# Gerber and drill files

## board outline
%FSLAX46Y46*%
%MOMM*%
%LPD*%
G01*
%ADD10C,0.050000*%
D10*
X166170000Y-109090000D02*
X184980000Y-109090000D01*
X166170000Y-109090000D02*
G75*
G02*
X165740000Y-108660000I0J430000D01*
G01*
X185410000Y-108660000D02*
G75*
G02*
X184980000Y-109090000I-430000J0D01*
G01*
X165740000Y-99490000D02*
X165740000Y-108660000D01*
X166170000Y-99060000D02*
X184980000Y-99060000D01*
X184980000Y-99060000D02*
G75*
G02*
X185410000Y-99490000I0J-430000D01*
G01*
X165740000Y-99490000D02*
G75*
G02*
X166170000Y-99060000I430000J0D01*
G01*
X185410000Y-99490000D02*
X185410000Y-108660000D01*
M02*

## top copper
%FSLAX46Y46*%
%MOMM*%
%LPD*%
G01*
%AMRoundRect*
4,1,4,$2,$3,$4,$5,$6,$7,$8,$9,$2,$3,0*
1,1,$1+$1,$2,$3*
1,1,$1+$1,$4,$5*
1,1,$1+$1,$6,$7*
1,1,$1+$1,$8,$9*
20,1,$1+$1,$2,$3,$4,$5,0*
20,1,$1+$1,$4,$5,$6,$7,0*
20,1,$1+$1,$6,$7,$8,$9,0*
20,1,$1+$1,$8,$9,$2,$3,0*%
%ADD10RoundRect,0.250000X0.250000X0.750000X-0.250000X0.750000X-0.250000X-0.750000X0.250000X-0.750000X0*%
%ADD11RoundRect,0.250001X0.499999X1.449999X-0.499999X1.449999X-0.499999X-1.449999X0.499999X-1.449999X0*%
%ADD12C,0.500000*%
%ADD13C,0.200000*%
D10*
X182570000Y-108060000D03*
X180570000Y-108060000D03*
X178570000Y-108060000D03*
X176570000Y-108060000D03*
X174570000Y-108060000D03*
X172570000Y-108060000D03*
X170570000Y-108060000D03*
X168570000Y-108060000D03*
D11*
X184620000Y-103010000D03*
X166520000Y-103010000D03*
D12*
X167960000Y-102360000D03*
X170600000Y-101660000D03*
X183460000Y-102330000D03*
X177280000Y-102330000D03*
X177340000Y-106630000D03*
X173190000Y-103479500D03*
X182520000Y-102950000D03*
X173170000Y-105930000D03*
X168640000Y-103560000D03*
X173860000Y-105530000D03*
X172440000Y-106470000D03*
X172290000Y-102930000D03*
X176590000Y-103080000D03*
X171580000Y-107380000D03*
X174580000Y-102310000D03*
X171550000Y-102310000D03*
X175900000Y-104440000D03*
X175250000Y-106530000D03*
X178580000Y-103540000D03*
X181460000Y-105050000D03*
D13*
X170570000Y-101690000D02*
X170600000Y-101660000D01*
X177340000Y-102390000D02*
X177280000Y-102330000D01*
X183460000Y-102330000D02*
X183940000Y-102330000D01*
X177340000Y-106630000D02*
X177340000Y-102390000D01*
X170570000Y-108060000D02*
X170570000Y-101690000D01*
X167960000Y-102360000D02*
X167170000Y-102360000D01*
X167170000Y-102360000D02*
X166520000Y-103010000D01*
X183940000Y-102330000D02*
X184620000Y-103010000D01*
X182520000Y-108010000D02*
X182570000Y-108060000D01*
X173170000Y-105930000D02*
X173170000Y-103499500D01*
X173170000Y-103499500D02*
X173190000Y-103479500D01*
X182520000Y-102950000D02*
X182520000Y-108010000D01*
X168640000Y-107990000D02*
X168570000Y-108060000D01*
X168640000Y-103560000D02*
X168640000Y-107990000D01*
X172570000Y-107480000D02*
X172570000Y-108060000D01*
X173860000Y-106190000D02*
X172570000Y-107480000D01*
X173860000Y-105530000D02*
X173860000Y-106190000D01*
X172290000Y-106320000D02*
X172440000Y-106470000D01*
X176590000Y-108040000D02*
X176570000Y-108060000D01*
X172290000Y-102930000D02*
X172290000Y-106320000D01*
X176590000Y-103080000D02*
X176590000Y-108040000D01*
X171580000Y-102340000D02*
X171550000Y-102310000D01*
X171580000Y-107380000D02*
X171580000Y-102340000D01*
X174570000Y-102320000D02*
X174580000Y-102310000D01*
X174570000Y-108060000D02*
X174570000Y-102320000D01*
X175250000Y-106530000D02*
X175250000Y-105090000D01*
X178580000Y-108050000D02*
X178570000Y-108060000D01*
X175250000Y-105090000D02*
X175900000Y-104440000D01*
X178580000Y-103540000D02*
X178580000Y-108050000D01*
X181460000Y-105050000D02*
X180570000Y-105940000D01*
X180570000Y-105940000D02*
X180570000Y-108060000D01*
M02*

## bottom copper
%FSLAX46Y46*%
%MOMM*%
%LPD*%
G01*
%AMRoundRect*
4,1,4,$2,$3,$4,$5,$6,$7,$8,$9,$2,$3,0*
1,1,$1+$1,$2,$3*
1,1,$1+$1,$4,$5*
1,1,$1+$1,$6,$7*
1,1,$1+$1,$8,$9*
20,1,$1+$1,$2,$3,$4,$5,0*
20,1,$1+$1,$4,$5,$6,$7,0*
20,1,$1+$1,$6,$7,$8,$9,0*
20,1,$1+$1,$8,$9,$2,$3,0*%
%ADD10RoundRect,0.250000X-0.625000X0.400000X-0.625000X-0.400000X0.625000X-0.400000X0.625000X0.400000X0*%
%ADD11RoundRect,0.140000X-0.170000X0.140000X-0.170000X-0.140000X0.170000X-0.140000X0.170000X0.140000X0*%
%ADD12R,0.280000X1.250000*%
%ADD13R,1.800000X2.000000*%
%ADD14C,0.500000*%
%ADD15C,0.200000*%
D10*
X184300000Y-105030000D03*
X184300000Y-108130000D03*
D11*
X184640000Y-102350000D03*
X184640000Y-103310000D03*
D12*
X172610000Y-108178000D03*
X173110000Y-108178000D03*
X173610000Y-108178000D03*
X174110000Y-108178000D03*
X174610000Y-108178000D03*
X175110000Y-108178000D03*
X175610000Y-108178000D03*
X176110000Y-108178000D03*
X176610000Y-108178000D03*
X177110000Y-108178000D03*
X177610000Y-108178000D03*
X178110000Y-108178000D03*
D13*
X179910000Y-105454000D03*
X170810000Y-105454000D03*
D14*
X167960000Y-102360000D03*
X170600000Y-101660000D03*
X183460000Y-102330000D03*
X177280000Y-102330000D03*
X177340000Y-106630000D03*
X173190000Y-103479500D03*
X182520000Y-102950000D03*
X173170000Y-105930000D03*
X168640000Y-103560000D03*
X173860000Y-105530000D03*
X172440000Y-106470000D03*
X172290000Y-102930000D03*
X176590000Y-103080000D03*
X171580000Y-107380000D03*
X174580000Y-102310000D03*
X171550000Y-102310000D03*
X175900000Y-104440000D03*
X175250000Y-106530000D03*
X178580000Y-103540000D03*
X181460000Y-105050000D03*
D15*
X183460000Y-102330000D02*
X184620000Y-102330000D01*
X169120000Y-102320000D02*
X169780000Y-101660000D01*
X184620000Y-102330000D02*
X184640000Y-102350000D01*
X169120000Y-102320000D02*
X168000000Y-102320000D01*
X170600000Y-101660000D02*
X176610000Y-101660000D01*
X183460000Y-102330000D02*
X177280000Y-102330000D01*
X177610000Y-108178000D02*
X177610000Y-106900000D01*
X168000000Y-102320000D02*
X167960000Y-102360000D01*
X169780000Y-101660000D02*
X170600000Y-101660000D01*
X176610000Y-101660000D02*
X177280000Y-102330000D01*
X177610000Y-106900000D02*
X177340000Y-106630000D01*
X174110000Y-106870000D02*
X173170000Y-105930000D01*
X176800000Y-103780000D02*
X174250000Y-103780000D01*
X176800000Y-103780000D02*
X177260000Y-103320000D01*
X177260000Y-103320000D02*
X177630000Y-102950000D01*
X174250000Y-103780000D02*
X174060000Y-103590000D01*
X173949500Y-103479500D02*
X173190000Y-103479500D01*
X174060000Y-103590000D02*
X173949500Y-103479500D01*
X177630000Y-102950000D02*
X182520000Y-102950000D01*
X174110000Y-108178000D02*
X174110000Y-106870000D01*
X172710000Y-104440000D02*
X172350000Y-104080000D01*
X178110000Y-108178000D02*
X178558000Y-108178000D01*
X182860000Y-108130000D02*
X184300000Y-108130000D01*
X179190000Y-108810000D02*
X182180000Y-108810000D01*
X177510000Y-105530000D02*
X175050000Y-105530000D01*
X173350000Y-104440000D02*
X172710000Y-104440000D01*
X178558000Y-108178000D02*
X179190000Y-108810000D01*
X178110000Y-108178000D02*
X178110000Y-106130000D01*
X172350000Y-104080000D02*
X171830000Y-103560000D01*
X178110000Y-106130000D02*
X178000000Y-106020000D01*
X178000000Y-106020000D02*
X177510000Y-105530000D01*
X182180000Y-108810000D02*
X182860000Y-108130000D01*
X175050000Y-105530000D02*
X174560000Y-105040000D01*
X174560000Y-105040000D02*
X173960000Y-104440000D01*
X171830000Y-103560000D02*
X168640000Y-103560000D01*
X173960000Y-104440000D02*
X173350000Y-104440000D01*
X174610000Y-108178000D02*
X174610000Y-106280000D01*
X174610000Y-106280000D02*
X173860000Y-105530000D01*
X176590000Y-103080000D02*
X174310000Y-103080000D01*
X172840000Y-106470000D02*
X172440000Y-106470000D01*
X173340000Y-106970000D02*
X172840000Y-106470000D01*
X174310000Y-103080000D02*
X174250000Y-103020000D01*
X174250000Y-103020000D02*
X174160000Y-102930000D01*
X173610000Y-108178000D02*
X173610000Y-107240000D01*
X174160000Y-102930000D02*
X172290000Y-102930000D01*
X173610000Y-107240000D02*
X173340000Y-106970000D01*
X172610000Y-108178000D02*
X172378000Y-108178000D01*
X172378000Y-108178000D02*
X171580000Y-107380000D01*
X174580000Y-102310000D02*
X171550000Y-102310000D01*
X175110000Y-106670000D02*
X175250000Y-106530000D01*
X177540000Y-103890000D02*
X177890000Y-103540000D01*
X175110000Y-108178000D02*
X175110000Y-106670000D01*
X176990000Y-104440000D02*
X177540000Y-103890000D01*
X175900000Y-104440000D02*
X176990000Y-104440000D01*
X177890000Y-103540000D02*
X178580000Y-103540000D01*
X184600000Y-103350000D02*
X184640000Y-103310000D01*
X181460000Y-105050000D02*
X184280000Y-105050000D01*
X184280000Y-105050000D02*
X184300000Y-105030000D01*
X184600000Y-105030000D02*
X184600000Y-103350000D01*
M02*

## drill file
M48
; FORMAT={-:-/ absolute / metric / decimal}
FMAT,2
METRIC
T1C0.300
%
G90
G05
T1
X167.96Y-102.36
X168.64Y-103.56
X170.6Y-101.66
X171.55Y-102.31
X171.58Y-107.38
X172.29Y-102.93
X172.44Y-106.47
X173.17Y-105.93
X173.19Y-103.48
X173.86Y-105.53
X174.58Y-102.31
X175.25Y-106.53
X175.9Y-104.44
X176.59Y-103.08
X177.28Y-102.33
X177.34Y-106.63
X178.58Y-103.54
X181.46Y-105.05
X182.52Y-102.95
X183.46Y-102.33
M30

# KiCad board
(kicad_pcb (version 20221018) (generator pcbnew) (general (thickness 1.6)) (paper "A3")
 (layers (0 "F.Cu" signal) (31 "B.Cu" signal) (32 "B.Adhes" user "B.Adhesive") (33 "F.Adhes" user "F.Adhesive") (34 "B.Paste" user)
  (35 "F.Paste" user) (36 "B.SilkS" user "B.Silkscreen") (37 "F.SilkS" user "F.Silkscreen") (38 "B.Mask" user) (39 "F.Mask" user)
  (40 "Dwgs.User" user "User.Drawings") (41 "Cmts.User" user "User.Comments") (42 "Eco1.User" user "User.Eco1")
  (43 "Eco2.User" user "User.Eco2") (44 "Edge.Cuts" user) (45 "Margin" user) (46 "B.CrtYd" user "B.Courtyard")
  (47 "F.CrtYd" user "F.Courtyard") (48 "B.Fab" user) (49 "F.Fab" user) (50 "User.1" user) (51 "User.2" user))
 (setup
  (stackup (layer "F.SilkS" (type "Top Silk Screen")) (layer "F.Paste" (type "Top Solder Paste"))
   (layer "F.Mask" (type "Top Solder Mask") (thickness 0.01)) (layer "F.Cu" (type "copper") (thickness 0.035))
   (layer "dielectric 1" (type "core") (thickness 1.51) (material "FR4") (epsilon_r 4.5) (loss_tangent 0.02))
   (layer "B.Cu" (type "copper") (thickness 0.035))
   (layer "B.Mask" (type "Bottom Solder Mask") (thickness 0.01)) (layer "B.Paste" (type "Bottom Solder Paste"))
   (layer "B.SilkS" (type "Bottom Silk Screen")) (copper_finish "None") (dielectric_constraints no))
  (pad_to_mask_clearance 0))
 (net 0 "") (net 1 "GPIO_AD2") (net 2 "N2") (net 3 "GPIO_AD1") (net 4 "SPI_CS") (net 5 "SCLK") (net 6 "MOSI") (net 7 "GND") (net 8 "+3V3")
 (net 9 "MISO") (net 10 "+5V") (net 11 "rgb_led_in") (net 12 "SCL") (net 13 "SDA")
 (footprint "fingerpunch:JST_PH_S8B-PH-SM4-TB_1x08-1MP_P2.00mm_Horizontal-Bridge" (layer "F.Cu") (at 175.57 105.16 180)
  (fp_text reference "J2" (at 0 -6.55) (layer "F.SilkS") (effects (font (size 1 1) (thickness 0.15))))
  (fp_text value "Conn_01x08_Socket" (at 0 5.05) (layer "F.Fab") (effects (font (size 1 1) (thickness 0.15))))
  (pad "1" smd roundrect (at -7 -2.9 180) (size 1 2) (layers "F.Cu" "F.Paste" "F.Mask") (roundrect_rratio 0.25) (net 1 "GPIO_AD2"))
  (pad "2" smd roundrect (at -5 -2.9 180) (size 1 2) (layers "F.Cu" "F.Paste" "F.Mask") (roundrect_rratio 0.25) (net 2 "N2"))
  (pad "3" smd roundrect (at -3 -2.9 180) (size 1 2) (layers "F.Cu" "F.Paste" "F.Mask") (roundrect_rratio 0.25) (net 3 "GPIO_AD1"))
  (pad "4" smd roundrect (at -1 -2.9 180) (size 1 2) (layers "F.Cu" "F.Paste" "F.Mask") (roundrect_rratio 0.25) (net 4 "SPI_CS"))
  (pad "5" smd roundrect (at 1 -2.9 180) (size 1 2) (layers "F.Cu" "F.Paste" "F.Mask") (roundrect_rratio 0.25) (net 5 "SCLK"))
  (pad "6" smd roundrect (at 3 -2.9 180) (size 1 2) (layers "F.Cu" "F.Paste" "F.Mask") (roundrect_rratio 0.25) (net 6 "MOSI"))
  (pad "7" smd roundrect (at 5 -2.9 180) (size 1 2) (layers "F.Cu" "F.Paste" "F.Mask") (roundrect_rratio 0.25) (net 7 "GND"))
  (pad "8" smd roundrect (at 7 -2.9 180) (size 1 2) (layers "F.Cu" "F.Paste" "F.Mask") (roundrect_rratio 0.25) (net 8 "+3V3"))
  (pad "9" smd roundrect (at -9.05 2.15 180) (size 1.5 3.4) (layers "F.Cu" "F.Paste" "F.Mask") (roundrect_rratio 0.1666673333) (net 7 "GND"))
  (pad "9" smd roundrect (at 9.05 2.15 180) (size 1.5 3.4) (layers "F.Cu" "F.Paste" "F.Mask") (roundrect_rratio 0.1666673333) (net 7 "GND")))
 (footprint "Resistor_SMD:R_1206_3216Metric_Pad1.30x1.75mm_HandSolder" (layer "B.Cu") (at 184.3 106.58 -90)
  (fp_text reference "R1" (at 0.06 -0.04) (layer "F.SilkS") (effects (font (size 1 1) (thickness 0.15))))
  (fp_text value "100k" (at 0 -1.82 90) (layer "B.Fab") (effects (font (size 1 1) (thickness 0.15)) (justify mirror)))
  (pad "1" smd roundrect (at -1.55 0 270) (size 1.3 1.75) (layers "B.Cu" "B.Paste" "B.Mask") (roundrect_rratio 0.1923076923) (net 2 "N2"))
  (pad "2" smd roundrect (at 1.55 0 270) (size 1.3 1.75) (layers "B.Cu" "B.Paste" "B.Mask") (roundrect_rratio 0.1923076923) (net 8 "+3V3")))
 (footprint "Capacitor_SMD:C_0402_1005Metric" (layer "B.Cu") (at 184.64 102.83 -90)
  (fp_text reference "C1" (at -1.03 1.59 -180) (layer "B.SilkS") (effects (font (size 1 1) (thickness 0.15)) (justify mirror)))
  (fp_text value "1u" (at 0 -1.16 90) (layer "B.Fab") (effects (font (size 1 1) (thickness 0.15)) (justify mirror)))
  (pad "1" smd roundrect (at -0.48 0 270) (size 0.56 0.62) (layers "B.Cu" "B.Paste" "B.Mask") (roundrect_rratio 0.25) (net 7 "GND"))
  (pad "2" smd roundrect (at 0.48 0 270) (size 0.56 0.62) (layers "B.Cu" "B.Paste" "B.Mask") (roundrect_rratio 0.25) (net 2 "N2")))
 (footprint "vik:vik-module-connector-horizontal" (layer "B.Cu") (at 175.36 106.14)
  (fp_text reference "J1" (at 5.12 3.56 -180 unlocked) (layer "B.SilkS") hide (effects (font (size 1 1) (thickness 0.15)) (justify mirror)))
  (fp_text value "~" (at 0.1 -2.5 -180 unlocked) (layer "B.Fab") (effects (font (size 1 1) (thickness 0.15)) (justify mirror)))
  (pad "1" smd rect (at -2.75 2.038) (size 0.28 1.25) (layers "B.Cu" "B.Paste" "B.Mask") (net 5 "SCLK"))
  (pad "2" smd rect (at -2.25 2.038) (size 0.28 1.25) (layers "B.Cu" "B.Paste" "B.Mask") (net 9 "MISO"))
  (pad "3" smd rect (at -1.75 2.038) (size 0.28 1.25) (layers "B.Cu" "B.Paste" "B.Mask") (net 4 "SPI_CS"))
  (pad "4" smd rect (at -1.25 2.038) (size 0.28 1.25) (layers "B.Cu" "B.Paste" "B.Mask") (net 1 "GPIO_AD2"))
  (pad "5" smd rect (at -0.75 2.038) (size 0.28 1.25) (layers "B.Cu" "B.Paste" "B.Mask") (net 6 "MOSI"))
  (pad "6" smd rect (at -0.25 2.038) (size 0.28 1.25) (layers "B.Cu" "B.Paste" "B.Mask") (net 3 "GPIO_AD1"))
  (pad "7" smd rect (at 0.25 2.038) (size 0.28 1.25) (layers "B.Cu" "B.Paste" "B.Mask") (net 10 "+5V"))
  (pad "8" smd rect (at 0.75 2.038) (size 0.28 1.25) (layers "B.Cu" "B.Paste" "B.Mask") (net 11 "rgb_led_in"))
  (pad "9" smd rect (at 1.25 2.038) (size 0.28 1.25) (layers "B.Cu" "B.Paste" "B.Mask") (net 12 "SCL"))
  (pad "10" smd rect (at 1.75 2.038) (size 0.28 1.25) (layers "B.Cu" "B.Paste" "B.Mask") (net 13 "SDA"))
  (pad "11" smd rect (at 2.25 2.038) (size 0.28 1.25) (layers "B.Cu" "B.Paste" "B.Mask") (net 7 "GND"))
  (pad "12" smd rect (at 2.75 2.038) (size 0.28 1.25) (layers "B.Cu" "B.Paste" "B.Mask") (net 8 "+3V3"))
  (pad "13" smd rect (at 4.55 -0.686) (size 1.8 2) (layers "B.Cu" "B.Paste" "B.Mask"))
  (pad "14" smd rect (at -4.55 -0.686) (size 1.8 2) (layers "B.Cu" "B.Paste" "B.Mask")))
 (gr_line (start 166.17 109.09) (end 184.98 109.09) (stroke (width 0.05) (type default)) (layer "Edge.Cuts"))
 (gr_arc (start 166.17 109.09) (mid 165.865944 108.964056) (end 165.74 108.66) (stroke (width 0.05) (type default)) (layer "Edge.Cuts"))
 (gr_arc (start 185.41 108.66) (mid 185.284056 108.964056) (end 184.98 109.09) (stroke (width 0.05) (type default)) (layer "Edge.Cuts"))
 (gr_line (start 165.74 99.49) (end 165.74 108.66) (stroke (width 0.05) (type default)) (layer "Edge.Cuts"))
 (gr_line (start 166.17 99.06) (end 184.98 99.06) (stroke (width 0.05) (type default)) (layer "Edge.Cuts"))
 (gr_arc (start 184.98 99.06) (mid 185.284056 99.185944) (end 185.41 99.49) (stroke (width 0.05) (type default)) (layer "Edge.Cuts"))
 (gr_arc (start 165.74 99.49) (mid 165.865944 99.185944) (end 166.17 99.06) (stroke (width 0.05) (type default)) (layer "Edge.Cuts"))
 (gr_line (start 185.41 99.49) (end 185.41 108.66) (stroke (width 0.05) (type default)) (layer "Edge.Cuts"))
 (segment (start 170.57 101.69) (end 170.6 101.66) (width 0.2) (layer "F.Cu") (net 7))
 (segment (start 177.34 102.39) (end 177.28 102.33) (width 0.2) (layer "F.Cu") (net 7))
 (segment (start 183.46 102.33) (end 183.94 102.33) (width 0.2) (layer "F.Cu") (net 7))
 (segment (start 177.34 106.63) (end 177.34 102.39) (width 0.2) (layer "F.Cu") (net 7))
 (segment (start 170.57 108.06) (end 170.57 101.69) (width 0.2) (layer "F.Cu") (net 7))
 (segment (start 167.96 102.36) (end 167.17 102.36) (width 0.2) (layer "F.Cu") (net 7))
 (segment (start 167.17 102.36) (end 166.52 103.01) (width 0.2) (layer "F.Cu") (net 7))
 (segment (start 183.94 102.33) (end 184.62 103.01) (width 0.2) (layer "F.Cu") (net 7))
 (via (at 167.96 102.36) (size 0.5) (drill 0.3) (layers "F.Cu" "B.Cu") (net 7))
 (via (at 170.6 101.66) (size 0.5) (drill 0.3) (layers "F.Cu" "B.Cu") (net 7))
 (via (at 183.46 102.33) (size 0.5) (drill 0.3) (layers "F.Cu" "B.Cu") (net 7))
 (via (at 177.28 102.33) (size 0.5) (drill 0.3) (layers "F.Cu" "B.Cu") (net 7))
 (via (at 177.34 106.63) (size 0.5) (drill 0.3) (layers "F.Cu" "B.Cu") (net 7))
 (segment (start 183.46 102.33) (end 184.62 102.33) (width 0.2) (layer "B.Cu") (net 7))
 (segment (start 169.12 102.32) (end 169.78 101.66) (width 0.2) (layer "B.Cu") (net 7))
 (segment (start 184.62 102.33) (end 184.64 102.35) (width 0.2) (layer "B.Cu") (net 7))
 (segment (start 169.12 102.32) (end 168 102.32) (width 0.2) (layer "B.Cu") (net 7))
 (segment (start 170.6 101.66) (end 176.61 101.66) (width 0.2) (layer "B.Cu") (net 7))
 (segment (start 183.46 102.33) (end 177.28 102.33) (width 0.2) (layer "B.Cu") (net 7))
 (segment (start 177.61 108.178) (end 177.61 106.9) (width 0.2) (layer "B.Cu") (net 7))
 (segment (start 168 102.32) (end 167.96 102.36) (width 0.2) (layer "B.Cu") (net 7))
 (segment (start 169.78 101.66) (end 170.6 101.66) (width 0.2) (layer "B.Cu") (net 7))
 (segment (start 176.61 101.66) (end 177.28 102.33) (width 0.2) (layer "B.Cu") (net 7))
 (segment (start 177.61 106.9) (end 177.34 106.63) (width 0.2) (layer "B.Cu") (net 7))
 (segment (start 182.52 108.01) (end 182.57 108.06) (width 0.2) (layer "F.Cu") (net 1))
 (segment (start 173.17 105.93) (end 173.17 103.4995) (width 0.2) (layer "F.Cu") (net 1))
 (segment (start 173.17 103.4995) (end 173.19 103.4795) (width 0.2) (layer "F.Cu") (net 1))
 (segment (start 182.52 102.95) (end 182.52 108.01) (width 0.2) (layer "F.Cu") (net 1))
 (via (at 173.19 103.4795) (size 0.5) (drill 0.3) (layers "F.Cu" "B.Cu") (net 1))
 (via (at 182.52 102.95) (size 0.5) (drill 0.3) (layers "F.Cu" "B.Cu") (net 1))
 (via (at 173.17 105.93) (size 0.5) (drill 0.3) (layers "F.Cu" "B.Cu") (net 1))
 (segment (start 174.11 106.87) (end 173.17 105.93) (width 0.2) (layer "B.Cu") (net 1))
 (segment (start 176.8 103.78) (end 174.25 103.78) (width 0.2) (layer "B.Cu") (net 1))
 (segment (start 176.8 103.78) (end 177.26 103.32) (width 0.2) (layer "B.Cu") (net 1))
 (segment (start 177.26 103.32) (end 177.63 102.95) (width 0.2) (layer "B.Cu") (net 1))
 (segment (start 174.25 103.78) (end 174.06 103.59) (width 0.2) (layer "B.Cu") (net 1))
 (segment (start 173.9495 103.4795) (end 173.19 103.4795) (width 0.2) (layer "B.Cu") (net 1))
 (segment (start 174.06 103.59) (end 173.9495 103.4795) (width 0.2) (layer "B.Cu") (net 1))
 (segment (start 177.63 102.95) (end 182.52 102.95) (width 0.2) (layer "B.Cu") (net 1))
 (segment (start 174.11 108.178) (end 174.11 106.87) (width 0.2) (layer "B.Cu") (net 1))
 (segment (start 168.64 107.99) (end 168.57 108.06) (width 0.2) (layer "F.Cu") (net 8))
 (segment (start 168.64 103.56) (end 168.64 107.99) (width 0.2) (layer "F.Cu") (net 8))
 (via (at 168.64 103.56) (size 0.5) (drill 0.3) (layers "F.Cu" "B.Cu") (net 8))
 (segment (start 172.71 104.44) (end 172.35 104.08) (width 0.2) (layer "B.Cu") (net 8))
 (segment (start 178.11 108.178) (end 178.558 108.178) (width 0.2) (layer "B.Cu") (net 8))
 (segment (start 182.86 108.13) (end 184.3 108.13) (width 0.2) (layer "B.Cu") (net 8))
 (segment (start 179.19 108.81) (end 182.18 108.81) (width 0.2) (layer "B.Cu") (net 8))
 (segment (start 177.51 105.53) (end 175.05 105.53) (width 0.2) (layer "B.Cu") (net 8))
 (segment (start 173.35 104.44) (end 172.71 104.44) (width 0.2) (layer "B.Cu") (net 8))
 (segment (start 178.558 108.178) (end 179.19 108.81) (width 0.2) (layer "B.Cu") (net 8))
 (segment (start 178.11 108.178) (end 178.11 106.13) (width 0.2) (layer "B.Cu") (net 8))
 (segment (start 172.35 104.08) (end 171.83 103.56) (width 0.2) (layer "B.Cu") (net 8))
 (segment (start 178.11 106.13) (end 178 106.02) (width 0.2) (layer "B.Cu") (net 8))
 (segment (start 178 106.02) (end 177.51 105.53) (width 0.2) (layer "B.Cu") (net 8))
 (segment (start 182.18 108.81) (end 182.86 108.13) (width 0.2) (layer "B.Cu") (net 8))
 (segment (start 175.05 105.53) (end 174.56 105.04) (width 0.2) (layer "B.Cu") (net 8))
 (segment (start 174.56 105.04) (end 173.96 104.44) (width 0.2) (layer "B.Cu") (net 8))
 (segment (start 171.83 103.56) (end 168.64 103.56) (width 0.2) (layer "B.Cu") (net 8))
 (segment (start 173.96 104.44) (end 173.35 104.44) (width 0.2) (layer "B.Cu") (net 8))
 (segment (start 172.57 107.48) (end 172.57 108.06) (width 0.2) (layer "F.Cu") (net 6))
 (segment (start 173.86 106.19) (end 172.57 107.48) (width 0.2) (layer "F.Cu") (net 6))
 (segment (start 173.86 105.53) (end 173.86 106.19) (width 0.2) (layer "F.Cu") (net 6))
 (via (at 173.86 105.53) (size 0.5) (drill 0.3) (layers "F.Cu" "B.Cu") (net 6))
 (segment (start 174.61 108.178) (end 174.61 106.28) (width 0.2) (layer "B.Cu") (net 6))
 (segment (start 174.61 106.28) (end 173.86 105.53) (width 0.2) (layer "B.Cu") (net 6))
 (segment (start 172.29 106.32) (end 172.44 106.47) (width 0.2) (layer "F.Cu") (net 4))
 (segment (start 176.59 108.04) (end 176.57 108.06) (width 0.2) (layer "F.Cu") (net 4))
 (segment (start 172.29 102.93) (end 172.29 106.32) (width 0.2) (layer "F.Cu") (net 4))
 (segment (start 176.59 103.08) (end 176.59 108.04) (width 0.2) (layer "F.Cu") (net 4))
 (via (at 172.44 106.47) (size 0.5) (drill 0.3) (layers "F.Cu" "B.Cu") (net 4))
 (via (at 172.29 102.93) (size 0.5) (drill 0.3) (layers "F.Cu" "B.Cu") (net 4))
 (via (at 176.59 103.08) (size 0.5) (drill 0.3) (layers "F.Cu" "B.Cu") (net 4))
 (segment (start 176.59 103.08) (end 174.31 103.08) (width 0.2) (layer "B.Cu") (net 4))
 (segment (start 172.84 106.47) (end 172.44 106.47) (width 0.2) (layer "B.Cu") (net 4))
 (segment (start 173.34 106.97) (end 172.84 106.47) (width 0.2) (layer "B.Cu") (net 4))
 (segment (start 174.31 103.08) (end 174.25 103.02) (width 0.2) (layer "B.Cu") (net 4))
 (segment (start 174.25 103.02) (end 174.16 102.93) (width 0.2) (layer "B.Cu") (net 4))
 (segment (start 173.61 108.178) (end 173.61 107.24) (width 0.2) (layer "B.Cu") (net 4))
 (segment (start 174.16 102.93) (end 172.29 102.93) (width 0.2) (layer "B.Cu") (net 4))
 (segment (start 173.61 107.24) (end 173.34 106.97) (width 0.2) (layer "B.Cu") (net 4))
 (segment (start 171.58 102.34) (end 171.55 102.31) (width 0.2) (layer "F.Cu") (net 5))
 (segment (start 171.58 107.38) (end 171.58 102.34) (width 0.2) (layer "F.Cu") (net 5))
 (segment (start 174.57 102.32) (end 174.58 102.31) (width 0.2) (layer "F.Cu") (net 5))
 (segment (start 174.57 108.06) (end 174.57 102.32) (width 0.2) (layer "F.Cu") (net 5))
 (via (at 171.58 107.38) (size 0.5) (drill 0.3) (layers "F.Cu" "B.Cu") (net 5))
 (via (at 174.58 102.31) (size 0.5) (drill 0.3) (layers "F.Cu" "B.Cu") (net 5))
 (via (at 171.55 102.31) (size 0.5) (drill 0.3) (layers "F.Cu" "B.Cu") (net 5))
 (segment (start 172.61 108.178) (end 172.378 108.178) (width 0.2) (layer "B.Cu") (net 5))
 (segment (start 172.378 108.178) (end 171.58 107.38) (width 0.2) (layer "B.Cu") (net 5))
 (segment (start 174.58 102.31) (end 171.55 102.31) (width 0.2) (layer "B.Cu") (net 5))
 (segment (start 175.25 106.53) (end 175.25 105.09) (width 0.2) (layer "F.Cu") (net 3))
 (segment (start 178.58 108.05) (end 178.57 108.06) (width 0.2) (layer "F.Cu") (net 3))
 (segment (start 175.25 105.09) (end 175.9 104.44) (width 0.2) (layer "F.Cu") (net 3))
 (segment (start 178.58 103.54) (end 178.58 108.05) (width 0.2) (layer "F.Cu") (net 3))
 (via (at 175.9 104.44) (size 0.5) (drill 0.3) (layers "F.Cu" "B.Cu") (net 3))
 (via (at 175.25 106.53) (size 0.5) (drill 0.3) (layers "F.Cu" "B.Cu") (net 3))
 (via (at 178.58 103.54) (size 0.5) (drill 0.3) (layers "F.Cu" "B.Cu") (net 3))
 (segment (start 175.11 106.67) (end 175.25 106.53) (width 0.2) (layer "B.Cu") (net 3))
 (segment (start 177.54 103.89) (end 177.89 103.54) (width 0.2) (layer "B.Cu") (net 3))
 (segment (start 175.11 108.178) (end 175.11 106.67) (width 0.2) (layer "B.Cu") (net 3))
 (segment (start 176.99 104.44) (end 177.54 103.89) (width 0.2) (layer "B.Cu") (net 3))
 (segment (start 175.9 104.44) (end 176.99 104.44) (width 0.2) (layer "B.Cu") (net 3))
 (segment (start 177.89 103.54) (end 178.58 103.54) (width 0.2) (layer "B.Cu") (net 3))
 (segment (start 181.46 105.05) (end 180.57 105.94) (width 0.2) (layer "F.Cu") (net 2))
 (segment (start 180.57 105.94) (end 180.57 108.06) (width 0.2) (layer "F.Cu") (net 2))
 (via (at 181.46 105.05) (size 0.5) (drill 0.3) (layers "F.Cu" "B.Cu") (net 2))
 (segment (start 184.6 103.35) (end 184.64 103.31) (width 0.2) (layer "B.Cu") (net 2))
 (segment (start 181.46 105.05) (end 184.28 105.05) (width 0.2) (layer "B.Cu") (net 2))
 (segment (start 184.28 105.05) (end 184.3 105.03) (width 0.2) (layer "B.Cu") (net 2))
 (segment (start 184.6 105.03) (end 184.6 103.35) (width 0.2) (layer "B.Cu") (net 2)))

